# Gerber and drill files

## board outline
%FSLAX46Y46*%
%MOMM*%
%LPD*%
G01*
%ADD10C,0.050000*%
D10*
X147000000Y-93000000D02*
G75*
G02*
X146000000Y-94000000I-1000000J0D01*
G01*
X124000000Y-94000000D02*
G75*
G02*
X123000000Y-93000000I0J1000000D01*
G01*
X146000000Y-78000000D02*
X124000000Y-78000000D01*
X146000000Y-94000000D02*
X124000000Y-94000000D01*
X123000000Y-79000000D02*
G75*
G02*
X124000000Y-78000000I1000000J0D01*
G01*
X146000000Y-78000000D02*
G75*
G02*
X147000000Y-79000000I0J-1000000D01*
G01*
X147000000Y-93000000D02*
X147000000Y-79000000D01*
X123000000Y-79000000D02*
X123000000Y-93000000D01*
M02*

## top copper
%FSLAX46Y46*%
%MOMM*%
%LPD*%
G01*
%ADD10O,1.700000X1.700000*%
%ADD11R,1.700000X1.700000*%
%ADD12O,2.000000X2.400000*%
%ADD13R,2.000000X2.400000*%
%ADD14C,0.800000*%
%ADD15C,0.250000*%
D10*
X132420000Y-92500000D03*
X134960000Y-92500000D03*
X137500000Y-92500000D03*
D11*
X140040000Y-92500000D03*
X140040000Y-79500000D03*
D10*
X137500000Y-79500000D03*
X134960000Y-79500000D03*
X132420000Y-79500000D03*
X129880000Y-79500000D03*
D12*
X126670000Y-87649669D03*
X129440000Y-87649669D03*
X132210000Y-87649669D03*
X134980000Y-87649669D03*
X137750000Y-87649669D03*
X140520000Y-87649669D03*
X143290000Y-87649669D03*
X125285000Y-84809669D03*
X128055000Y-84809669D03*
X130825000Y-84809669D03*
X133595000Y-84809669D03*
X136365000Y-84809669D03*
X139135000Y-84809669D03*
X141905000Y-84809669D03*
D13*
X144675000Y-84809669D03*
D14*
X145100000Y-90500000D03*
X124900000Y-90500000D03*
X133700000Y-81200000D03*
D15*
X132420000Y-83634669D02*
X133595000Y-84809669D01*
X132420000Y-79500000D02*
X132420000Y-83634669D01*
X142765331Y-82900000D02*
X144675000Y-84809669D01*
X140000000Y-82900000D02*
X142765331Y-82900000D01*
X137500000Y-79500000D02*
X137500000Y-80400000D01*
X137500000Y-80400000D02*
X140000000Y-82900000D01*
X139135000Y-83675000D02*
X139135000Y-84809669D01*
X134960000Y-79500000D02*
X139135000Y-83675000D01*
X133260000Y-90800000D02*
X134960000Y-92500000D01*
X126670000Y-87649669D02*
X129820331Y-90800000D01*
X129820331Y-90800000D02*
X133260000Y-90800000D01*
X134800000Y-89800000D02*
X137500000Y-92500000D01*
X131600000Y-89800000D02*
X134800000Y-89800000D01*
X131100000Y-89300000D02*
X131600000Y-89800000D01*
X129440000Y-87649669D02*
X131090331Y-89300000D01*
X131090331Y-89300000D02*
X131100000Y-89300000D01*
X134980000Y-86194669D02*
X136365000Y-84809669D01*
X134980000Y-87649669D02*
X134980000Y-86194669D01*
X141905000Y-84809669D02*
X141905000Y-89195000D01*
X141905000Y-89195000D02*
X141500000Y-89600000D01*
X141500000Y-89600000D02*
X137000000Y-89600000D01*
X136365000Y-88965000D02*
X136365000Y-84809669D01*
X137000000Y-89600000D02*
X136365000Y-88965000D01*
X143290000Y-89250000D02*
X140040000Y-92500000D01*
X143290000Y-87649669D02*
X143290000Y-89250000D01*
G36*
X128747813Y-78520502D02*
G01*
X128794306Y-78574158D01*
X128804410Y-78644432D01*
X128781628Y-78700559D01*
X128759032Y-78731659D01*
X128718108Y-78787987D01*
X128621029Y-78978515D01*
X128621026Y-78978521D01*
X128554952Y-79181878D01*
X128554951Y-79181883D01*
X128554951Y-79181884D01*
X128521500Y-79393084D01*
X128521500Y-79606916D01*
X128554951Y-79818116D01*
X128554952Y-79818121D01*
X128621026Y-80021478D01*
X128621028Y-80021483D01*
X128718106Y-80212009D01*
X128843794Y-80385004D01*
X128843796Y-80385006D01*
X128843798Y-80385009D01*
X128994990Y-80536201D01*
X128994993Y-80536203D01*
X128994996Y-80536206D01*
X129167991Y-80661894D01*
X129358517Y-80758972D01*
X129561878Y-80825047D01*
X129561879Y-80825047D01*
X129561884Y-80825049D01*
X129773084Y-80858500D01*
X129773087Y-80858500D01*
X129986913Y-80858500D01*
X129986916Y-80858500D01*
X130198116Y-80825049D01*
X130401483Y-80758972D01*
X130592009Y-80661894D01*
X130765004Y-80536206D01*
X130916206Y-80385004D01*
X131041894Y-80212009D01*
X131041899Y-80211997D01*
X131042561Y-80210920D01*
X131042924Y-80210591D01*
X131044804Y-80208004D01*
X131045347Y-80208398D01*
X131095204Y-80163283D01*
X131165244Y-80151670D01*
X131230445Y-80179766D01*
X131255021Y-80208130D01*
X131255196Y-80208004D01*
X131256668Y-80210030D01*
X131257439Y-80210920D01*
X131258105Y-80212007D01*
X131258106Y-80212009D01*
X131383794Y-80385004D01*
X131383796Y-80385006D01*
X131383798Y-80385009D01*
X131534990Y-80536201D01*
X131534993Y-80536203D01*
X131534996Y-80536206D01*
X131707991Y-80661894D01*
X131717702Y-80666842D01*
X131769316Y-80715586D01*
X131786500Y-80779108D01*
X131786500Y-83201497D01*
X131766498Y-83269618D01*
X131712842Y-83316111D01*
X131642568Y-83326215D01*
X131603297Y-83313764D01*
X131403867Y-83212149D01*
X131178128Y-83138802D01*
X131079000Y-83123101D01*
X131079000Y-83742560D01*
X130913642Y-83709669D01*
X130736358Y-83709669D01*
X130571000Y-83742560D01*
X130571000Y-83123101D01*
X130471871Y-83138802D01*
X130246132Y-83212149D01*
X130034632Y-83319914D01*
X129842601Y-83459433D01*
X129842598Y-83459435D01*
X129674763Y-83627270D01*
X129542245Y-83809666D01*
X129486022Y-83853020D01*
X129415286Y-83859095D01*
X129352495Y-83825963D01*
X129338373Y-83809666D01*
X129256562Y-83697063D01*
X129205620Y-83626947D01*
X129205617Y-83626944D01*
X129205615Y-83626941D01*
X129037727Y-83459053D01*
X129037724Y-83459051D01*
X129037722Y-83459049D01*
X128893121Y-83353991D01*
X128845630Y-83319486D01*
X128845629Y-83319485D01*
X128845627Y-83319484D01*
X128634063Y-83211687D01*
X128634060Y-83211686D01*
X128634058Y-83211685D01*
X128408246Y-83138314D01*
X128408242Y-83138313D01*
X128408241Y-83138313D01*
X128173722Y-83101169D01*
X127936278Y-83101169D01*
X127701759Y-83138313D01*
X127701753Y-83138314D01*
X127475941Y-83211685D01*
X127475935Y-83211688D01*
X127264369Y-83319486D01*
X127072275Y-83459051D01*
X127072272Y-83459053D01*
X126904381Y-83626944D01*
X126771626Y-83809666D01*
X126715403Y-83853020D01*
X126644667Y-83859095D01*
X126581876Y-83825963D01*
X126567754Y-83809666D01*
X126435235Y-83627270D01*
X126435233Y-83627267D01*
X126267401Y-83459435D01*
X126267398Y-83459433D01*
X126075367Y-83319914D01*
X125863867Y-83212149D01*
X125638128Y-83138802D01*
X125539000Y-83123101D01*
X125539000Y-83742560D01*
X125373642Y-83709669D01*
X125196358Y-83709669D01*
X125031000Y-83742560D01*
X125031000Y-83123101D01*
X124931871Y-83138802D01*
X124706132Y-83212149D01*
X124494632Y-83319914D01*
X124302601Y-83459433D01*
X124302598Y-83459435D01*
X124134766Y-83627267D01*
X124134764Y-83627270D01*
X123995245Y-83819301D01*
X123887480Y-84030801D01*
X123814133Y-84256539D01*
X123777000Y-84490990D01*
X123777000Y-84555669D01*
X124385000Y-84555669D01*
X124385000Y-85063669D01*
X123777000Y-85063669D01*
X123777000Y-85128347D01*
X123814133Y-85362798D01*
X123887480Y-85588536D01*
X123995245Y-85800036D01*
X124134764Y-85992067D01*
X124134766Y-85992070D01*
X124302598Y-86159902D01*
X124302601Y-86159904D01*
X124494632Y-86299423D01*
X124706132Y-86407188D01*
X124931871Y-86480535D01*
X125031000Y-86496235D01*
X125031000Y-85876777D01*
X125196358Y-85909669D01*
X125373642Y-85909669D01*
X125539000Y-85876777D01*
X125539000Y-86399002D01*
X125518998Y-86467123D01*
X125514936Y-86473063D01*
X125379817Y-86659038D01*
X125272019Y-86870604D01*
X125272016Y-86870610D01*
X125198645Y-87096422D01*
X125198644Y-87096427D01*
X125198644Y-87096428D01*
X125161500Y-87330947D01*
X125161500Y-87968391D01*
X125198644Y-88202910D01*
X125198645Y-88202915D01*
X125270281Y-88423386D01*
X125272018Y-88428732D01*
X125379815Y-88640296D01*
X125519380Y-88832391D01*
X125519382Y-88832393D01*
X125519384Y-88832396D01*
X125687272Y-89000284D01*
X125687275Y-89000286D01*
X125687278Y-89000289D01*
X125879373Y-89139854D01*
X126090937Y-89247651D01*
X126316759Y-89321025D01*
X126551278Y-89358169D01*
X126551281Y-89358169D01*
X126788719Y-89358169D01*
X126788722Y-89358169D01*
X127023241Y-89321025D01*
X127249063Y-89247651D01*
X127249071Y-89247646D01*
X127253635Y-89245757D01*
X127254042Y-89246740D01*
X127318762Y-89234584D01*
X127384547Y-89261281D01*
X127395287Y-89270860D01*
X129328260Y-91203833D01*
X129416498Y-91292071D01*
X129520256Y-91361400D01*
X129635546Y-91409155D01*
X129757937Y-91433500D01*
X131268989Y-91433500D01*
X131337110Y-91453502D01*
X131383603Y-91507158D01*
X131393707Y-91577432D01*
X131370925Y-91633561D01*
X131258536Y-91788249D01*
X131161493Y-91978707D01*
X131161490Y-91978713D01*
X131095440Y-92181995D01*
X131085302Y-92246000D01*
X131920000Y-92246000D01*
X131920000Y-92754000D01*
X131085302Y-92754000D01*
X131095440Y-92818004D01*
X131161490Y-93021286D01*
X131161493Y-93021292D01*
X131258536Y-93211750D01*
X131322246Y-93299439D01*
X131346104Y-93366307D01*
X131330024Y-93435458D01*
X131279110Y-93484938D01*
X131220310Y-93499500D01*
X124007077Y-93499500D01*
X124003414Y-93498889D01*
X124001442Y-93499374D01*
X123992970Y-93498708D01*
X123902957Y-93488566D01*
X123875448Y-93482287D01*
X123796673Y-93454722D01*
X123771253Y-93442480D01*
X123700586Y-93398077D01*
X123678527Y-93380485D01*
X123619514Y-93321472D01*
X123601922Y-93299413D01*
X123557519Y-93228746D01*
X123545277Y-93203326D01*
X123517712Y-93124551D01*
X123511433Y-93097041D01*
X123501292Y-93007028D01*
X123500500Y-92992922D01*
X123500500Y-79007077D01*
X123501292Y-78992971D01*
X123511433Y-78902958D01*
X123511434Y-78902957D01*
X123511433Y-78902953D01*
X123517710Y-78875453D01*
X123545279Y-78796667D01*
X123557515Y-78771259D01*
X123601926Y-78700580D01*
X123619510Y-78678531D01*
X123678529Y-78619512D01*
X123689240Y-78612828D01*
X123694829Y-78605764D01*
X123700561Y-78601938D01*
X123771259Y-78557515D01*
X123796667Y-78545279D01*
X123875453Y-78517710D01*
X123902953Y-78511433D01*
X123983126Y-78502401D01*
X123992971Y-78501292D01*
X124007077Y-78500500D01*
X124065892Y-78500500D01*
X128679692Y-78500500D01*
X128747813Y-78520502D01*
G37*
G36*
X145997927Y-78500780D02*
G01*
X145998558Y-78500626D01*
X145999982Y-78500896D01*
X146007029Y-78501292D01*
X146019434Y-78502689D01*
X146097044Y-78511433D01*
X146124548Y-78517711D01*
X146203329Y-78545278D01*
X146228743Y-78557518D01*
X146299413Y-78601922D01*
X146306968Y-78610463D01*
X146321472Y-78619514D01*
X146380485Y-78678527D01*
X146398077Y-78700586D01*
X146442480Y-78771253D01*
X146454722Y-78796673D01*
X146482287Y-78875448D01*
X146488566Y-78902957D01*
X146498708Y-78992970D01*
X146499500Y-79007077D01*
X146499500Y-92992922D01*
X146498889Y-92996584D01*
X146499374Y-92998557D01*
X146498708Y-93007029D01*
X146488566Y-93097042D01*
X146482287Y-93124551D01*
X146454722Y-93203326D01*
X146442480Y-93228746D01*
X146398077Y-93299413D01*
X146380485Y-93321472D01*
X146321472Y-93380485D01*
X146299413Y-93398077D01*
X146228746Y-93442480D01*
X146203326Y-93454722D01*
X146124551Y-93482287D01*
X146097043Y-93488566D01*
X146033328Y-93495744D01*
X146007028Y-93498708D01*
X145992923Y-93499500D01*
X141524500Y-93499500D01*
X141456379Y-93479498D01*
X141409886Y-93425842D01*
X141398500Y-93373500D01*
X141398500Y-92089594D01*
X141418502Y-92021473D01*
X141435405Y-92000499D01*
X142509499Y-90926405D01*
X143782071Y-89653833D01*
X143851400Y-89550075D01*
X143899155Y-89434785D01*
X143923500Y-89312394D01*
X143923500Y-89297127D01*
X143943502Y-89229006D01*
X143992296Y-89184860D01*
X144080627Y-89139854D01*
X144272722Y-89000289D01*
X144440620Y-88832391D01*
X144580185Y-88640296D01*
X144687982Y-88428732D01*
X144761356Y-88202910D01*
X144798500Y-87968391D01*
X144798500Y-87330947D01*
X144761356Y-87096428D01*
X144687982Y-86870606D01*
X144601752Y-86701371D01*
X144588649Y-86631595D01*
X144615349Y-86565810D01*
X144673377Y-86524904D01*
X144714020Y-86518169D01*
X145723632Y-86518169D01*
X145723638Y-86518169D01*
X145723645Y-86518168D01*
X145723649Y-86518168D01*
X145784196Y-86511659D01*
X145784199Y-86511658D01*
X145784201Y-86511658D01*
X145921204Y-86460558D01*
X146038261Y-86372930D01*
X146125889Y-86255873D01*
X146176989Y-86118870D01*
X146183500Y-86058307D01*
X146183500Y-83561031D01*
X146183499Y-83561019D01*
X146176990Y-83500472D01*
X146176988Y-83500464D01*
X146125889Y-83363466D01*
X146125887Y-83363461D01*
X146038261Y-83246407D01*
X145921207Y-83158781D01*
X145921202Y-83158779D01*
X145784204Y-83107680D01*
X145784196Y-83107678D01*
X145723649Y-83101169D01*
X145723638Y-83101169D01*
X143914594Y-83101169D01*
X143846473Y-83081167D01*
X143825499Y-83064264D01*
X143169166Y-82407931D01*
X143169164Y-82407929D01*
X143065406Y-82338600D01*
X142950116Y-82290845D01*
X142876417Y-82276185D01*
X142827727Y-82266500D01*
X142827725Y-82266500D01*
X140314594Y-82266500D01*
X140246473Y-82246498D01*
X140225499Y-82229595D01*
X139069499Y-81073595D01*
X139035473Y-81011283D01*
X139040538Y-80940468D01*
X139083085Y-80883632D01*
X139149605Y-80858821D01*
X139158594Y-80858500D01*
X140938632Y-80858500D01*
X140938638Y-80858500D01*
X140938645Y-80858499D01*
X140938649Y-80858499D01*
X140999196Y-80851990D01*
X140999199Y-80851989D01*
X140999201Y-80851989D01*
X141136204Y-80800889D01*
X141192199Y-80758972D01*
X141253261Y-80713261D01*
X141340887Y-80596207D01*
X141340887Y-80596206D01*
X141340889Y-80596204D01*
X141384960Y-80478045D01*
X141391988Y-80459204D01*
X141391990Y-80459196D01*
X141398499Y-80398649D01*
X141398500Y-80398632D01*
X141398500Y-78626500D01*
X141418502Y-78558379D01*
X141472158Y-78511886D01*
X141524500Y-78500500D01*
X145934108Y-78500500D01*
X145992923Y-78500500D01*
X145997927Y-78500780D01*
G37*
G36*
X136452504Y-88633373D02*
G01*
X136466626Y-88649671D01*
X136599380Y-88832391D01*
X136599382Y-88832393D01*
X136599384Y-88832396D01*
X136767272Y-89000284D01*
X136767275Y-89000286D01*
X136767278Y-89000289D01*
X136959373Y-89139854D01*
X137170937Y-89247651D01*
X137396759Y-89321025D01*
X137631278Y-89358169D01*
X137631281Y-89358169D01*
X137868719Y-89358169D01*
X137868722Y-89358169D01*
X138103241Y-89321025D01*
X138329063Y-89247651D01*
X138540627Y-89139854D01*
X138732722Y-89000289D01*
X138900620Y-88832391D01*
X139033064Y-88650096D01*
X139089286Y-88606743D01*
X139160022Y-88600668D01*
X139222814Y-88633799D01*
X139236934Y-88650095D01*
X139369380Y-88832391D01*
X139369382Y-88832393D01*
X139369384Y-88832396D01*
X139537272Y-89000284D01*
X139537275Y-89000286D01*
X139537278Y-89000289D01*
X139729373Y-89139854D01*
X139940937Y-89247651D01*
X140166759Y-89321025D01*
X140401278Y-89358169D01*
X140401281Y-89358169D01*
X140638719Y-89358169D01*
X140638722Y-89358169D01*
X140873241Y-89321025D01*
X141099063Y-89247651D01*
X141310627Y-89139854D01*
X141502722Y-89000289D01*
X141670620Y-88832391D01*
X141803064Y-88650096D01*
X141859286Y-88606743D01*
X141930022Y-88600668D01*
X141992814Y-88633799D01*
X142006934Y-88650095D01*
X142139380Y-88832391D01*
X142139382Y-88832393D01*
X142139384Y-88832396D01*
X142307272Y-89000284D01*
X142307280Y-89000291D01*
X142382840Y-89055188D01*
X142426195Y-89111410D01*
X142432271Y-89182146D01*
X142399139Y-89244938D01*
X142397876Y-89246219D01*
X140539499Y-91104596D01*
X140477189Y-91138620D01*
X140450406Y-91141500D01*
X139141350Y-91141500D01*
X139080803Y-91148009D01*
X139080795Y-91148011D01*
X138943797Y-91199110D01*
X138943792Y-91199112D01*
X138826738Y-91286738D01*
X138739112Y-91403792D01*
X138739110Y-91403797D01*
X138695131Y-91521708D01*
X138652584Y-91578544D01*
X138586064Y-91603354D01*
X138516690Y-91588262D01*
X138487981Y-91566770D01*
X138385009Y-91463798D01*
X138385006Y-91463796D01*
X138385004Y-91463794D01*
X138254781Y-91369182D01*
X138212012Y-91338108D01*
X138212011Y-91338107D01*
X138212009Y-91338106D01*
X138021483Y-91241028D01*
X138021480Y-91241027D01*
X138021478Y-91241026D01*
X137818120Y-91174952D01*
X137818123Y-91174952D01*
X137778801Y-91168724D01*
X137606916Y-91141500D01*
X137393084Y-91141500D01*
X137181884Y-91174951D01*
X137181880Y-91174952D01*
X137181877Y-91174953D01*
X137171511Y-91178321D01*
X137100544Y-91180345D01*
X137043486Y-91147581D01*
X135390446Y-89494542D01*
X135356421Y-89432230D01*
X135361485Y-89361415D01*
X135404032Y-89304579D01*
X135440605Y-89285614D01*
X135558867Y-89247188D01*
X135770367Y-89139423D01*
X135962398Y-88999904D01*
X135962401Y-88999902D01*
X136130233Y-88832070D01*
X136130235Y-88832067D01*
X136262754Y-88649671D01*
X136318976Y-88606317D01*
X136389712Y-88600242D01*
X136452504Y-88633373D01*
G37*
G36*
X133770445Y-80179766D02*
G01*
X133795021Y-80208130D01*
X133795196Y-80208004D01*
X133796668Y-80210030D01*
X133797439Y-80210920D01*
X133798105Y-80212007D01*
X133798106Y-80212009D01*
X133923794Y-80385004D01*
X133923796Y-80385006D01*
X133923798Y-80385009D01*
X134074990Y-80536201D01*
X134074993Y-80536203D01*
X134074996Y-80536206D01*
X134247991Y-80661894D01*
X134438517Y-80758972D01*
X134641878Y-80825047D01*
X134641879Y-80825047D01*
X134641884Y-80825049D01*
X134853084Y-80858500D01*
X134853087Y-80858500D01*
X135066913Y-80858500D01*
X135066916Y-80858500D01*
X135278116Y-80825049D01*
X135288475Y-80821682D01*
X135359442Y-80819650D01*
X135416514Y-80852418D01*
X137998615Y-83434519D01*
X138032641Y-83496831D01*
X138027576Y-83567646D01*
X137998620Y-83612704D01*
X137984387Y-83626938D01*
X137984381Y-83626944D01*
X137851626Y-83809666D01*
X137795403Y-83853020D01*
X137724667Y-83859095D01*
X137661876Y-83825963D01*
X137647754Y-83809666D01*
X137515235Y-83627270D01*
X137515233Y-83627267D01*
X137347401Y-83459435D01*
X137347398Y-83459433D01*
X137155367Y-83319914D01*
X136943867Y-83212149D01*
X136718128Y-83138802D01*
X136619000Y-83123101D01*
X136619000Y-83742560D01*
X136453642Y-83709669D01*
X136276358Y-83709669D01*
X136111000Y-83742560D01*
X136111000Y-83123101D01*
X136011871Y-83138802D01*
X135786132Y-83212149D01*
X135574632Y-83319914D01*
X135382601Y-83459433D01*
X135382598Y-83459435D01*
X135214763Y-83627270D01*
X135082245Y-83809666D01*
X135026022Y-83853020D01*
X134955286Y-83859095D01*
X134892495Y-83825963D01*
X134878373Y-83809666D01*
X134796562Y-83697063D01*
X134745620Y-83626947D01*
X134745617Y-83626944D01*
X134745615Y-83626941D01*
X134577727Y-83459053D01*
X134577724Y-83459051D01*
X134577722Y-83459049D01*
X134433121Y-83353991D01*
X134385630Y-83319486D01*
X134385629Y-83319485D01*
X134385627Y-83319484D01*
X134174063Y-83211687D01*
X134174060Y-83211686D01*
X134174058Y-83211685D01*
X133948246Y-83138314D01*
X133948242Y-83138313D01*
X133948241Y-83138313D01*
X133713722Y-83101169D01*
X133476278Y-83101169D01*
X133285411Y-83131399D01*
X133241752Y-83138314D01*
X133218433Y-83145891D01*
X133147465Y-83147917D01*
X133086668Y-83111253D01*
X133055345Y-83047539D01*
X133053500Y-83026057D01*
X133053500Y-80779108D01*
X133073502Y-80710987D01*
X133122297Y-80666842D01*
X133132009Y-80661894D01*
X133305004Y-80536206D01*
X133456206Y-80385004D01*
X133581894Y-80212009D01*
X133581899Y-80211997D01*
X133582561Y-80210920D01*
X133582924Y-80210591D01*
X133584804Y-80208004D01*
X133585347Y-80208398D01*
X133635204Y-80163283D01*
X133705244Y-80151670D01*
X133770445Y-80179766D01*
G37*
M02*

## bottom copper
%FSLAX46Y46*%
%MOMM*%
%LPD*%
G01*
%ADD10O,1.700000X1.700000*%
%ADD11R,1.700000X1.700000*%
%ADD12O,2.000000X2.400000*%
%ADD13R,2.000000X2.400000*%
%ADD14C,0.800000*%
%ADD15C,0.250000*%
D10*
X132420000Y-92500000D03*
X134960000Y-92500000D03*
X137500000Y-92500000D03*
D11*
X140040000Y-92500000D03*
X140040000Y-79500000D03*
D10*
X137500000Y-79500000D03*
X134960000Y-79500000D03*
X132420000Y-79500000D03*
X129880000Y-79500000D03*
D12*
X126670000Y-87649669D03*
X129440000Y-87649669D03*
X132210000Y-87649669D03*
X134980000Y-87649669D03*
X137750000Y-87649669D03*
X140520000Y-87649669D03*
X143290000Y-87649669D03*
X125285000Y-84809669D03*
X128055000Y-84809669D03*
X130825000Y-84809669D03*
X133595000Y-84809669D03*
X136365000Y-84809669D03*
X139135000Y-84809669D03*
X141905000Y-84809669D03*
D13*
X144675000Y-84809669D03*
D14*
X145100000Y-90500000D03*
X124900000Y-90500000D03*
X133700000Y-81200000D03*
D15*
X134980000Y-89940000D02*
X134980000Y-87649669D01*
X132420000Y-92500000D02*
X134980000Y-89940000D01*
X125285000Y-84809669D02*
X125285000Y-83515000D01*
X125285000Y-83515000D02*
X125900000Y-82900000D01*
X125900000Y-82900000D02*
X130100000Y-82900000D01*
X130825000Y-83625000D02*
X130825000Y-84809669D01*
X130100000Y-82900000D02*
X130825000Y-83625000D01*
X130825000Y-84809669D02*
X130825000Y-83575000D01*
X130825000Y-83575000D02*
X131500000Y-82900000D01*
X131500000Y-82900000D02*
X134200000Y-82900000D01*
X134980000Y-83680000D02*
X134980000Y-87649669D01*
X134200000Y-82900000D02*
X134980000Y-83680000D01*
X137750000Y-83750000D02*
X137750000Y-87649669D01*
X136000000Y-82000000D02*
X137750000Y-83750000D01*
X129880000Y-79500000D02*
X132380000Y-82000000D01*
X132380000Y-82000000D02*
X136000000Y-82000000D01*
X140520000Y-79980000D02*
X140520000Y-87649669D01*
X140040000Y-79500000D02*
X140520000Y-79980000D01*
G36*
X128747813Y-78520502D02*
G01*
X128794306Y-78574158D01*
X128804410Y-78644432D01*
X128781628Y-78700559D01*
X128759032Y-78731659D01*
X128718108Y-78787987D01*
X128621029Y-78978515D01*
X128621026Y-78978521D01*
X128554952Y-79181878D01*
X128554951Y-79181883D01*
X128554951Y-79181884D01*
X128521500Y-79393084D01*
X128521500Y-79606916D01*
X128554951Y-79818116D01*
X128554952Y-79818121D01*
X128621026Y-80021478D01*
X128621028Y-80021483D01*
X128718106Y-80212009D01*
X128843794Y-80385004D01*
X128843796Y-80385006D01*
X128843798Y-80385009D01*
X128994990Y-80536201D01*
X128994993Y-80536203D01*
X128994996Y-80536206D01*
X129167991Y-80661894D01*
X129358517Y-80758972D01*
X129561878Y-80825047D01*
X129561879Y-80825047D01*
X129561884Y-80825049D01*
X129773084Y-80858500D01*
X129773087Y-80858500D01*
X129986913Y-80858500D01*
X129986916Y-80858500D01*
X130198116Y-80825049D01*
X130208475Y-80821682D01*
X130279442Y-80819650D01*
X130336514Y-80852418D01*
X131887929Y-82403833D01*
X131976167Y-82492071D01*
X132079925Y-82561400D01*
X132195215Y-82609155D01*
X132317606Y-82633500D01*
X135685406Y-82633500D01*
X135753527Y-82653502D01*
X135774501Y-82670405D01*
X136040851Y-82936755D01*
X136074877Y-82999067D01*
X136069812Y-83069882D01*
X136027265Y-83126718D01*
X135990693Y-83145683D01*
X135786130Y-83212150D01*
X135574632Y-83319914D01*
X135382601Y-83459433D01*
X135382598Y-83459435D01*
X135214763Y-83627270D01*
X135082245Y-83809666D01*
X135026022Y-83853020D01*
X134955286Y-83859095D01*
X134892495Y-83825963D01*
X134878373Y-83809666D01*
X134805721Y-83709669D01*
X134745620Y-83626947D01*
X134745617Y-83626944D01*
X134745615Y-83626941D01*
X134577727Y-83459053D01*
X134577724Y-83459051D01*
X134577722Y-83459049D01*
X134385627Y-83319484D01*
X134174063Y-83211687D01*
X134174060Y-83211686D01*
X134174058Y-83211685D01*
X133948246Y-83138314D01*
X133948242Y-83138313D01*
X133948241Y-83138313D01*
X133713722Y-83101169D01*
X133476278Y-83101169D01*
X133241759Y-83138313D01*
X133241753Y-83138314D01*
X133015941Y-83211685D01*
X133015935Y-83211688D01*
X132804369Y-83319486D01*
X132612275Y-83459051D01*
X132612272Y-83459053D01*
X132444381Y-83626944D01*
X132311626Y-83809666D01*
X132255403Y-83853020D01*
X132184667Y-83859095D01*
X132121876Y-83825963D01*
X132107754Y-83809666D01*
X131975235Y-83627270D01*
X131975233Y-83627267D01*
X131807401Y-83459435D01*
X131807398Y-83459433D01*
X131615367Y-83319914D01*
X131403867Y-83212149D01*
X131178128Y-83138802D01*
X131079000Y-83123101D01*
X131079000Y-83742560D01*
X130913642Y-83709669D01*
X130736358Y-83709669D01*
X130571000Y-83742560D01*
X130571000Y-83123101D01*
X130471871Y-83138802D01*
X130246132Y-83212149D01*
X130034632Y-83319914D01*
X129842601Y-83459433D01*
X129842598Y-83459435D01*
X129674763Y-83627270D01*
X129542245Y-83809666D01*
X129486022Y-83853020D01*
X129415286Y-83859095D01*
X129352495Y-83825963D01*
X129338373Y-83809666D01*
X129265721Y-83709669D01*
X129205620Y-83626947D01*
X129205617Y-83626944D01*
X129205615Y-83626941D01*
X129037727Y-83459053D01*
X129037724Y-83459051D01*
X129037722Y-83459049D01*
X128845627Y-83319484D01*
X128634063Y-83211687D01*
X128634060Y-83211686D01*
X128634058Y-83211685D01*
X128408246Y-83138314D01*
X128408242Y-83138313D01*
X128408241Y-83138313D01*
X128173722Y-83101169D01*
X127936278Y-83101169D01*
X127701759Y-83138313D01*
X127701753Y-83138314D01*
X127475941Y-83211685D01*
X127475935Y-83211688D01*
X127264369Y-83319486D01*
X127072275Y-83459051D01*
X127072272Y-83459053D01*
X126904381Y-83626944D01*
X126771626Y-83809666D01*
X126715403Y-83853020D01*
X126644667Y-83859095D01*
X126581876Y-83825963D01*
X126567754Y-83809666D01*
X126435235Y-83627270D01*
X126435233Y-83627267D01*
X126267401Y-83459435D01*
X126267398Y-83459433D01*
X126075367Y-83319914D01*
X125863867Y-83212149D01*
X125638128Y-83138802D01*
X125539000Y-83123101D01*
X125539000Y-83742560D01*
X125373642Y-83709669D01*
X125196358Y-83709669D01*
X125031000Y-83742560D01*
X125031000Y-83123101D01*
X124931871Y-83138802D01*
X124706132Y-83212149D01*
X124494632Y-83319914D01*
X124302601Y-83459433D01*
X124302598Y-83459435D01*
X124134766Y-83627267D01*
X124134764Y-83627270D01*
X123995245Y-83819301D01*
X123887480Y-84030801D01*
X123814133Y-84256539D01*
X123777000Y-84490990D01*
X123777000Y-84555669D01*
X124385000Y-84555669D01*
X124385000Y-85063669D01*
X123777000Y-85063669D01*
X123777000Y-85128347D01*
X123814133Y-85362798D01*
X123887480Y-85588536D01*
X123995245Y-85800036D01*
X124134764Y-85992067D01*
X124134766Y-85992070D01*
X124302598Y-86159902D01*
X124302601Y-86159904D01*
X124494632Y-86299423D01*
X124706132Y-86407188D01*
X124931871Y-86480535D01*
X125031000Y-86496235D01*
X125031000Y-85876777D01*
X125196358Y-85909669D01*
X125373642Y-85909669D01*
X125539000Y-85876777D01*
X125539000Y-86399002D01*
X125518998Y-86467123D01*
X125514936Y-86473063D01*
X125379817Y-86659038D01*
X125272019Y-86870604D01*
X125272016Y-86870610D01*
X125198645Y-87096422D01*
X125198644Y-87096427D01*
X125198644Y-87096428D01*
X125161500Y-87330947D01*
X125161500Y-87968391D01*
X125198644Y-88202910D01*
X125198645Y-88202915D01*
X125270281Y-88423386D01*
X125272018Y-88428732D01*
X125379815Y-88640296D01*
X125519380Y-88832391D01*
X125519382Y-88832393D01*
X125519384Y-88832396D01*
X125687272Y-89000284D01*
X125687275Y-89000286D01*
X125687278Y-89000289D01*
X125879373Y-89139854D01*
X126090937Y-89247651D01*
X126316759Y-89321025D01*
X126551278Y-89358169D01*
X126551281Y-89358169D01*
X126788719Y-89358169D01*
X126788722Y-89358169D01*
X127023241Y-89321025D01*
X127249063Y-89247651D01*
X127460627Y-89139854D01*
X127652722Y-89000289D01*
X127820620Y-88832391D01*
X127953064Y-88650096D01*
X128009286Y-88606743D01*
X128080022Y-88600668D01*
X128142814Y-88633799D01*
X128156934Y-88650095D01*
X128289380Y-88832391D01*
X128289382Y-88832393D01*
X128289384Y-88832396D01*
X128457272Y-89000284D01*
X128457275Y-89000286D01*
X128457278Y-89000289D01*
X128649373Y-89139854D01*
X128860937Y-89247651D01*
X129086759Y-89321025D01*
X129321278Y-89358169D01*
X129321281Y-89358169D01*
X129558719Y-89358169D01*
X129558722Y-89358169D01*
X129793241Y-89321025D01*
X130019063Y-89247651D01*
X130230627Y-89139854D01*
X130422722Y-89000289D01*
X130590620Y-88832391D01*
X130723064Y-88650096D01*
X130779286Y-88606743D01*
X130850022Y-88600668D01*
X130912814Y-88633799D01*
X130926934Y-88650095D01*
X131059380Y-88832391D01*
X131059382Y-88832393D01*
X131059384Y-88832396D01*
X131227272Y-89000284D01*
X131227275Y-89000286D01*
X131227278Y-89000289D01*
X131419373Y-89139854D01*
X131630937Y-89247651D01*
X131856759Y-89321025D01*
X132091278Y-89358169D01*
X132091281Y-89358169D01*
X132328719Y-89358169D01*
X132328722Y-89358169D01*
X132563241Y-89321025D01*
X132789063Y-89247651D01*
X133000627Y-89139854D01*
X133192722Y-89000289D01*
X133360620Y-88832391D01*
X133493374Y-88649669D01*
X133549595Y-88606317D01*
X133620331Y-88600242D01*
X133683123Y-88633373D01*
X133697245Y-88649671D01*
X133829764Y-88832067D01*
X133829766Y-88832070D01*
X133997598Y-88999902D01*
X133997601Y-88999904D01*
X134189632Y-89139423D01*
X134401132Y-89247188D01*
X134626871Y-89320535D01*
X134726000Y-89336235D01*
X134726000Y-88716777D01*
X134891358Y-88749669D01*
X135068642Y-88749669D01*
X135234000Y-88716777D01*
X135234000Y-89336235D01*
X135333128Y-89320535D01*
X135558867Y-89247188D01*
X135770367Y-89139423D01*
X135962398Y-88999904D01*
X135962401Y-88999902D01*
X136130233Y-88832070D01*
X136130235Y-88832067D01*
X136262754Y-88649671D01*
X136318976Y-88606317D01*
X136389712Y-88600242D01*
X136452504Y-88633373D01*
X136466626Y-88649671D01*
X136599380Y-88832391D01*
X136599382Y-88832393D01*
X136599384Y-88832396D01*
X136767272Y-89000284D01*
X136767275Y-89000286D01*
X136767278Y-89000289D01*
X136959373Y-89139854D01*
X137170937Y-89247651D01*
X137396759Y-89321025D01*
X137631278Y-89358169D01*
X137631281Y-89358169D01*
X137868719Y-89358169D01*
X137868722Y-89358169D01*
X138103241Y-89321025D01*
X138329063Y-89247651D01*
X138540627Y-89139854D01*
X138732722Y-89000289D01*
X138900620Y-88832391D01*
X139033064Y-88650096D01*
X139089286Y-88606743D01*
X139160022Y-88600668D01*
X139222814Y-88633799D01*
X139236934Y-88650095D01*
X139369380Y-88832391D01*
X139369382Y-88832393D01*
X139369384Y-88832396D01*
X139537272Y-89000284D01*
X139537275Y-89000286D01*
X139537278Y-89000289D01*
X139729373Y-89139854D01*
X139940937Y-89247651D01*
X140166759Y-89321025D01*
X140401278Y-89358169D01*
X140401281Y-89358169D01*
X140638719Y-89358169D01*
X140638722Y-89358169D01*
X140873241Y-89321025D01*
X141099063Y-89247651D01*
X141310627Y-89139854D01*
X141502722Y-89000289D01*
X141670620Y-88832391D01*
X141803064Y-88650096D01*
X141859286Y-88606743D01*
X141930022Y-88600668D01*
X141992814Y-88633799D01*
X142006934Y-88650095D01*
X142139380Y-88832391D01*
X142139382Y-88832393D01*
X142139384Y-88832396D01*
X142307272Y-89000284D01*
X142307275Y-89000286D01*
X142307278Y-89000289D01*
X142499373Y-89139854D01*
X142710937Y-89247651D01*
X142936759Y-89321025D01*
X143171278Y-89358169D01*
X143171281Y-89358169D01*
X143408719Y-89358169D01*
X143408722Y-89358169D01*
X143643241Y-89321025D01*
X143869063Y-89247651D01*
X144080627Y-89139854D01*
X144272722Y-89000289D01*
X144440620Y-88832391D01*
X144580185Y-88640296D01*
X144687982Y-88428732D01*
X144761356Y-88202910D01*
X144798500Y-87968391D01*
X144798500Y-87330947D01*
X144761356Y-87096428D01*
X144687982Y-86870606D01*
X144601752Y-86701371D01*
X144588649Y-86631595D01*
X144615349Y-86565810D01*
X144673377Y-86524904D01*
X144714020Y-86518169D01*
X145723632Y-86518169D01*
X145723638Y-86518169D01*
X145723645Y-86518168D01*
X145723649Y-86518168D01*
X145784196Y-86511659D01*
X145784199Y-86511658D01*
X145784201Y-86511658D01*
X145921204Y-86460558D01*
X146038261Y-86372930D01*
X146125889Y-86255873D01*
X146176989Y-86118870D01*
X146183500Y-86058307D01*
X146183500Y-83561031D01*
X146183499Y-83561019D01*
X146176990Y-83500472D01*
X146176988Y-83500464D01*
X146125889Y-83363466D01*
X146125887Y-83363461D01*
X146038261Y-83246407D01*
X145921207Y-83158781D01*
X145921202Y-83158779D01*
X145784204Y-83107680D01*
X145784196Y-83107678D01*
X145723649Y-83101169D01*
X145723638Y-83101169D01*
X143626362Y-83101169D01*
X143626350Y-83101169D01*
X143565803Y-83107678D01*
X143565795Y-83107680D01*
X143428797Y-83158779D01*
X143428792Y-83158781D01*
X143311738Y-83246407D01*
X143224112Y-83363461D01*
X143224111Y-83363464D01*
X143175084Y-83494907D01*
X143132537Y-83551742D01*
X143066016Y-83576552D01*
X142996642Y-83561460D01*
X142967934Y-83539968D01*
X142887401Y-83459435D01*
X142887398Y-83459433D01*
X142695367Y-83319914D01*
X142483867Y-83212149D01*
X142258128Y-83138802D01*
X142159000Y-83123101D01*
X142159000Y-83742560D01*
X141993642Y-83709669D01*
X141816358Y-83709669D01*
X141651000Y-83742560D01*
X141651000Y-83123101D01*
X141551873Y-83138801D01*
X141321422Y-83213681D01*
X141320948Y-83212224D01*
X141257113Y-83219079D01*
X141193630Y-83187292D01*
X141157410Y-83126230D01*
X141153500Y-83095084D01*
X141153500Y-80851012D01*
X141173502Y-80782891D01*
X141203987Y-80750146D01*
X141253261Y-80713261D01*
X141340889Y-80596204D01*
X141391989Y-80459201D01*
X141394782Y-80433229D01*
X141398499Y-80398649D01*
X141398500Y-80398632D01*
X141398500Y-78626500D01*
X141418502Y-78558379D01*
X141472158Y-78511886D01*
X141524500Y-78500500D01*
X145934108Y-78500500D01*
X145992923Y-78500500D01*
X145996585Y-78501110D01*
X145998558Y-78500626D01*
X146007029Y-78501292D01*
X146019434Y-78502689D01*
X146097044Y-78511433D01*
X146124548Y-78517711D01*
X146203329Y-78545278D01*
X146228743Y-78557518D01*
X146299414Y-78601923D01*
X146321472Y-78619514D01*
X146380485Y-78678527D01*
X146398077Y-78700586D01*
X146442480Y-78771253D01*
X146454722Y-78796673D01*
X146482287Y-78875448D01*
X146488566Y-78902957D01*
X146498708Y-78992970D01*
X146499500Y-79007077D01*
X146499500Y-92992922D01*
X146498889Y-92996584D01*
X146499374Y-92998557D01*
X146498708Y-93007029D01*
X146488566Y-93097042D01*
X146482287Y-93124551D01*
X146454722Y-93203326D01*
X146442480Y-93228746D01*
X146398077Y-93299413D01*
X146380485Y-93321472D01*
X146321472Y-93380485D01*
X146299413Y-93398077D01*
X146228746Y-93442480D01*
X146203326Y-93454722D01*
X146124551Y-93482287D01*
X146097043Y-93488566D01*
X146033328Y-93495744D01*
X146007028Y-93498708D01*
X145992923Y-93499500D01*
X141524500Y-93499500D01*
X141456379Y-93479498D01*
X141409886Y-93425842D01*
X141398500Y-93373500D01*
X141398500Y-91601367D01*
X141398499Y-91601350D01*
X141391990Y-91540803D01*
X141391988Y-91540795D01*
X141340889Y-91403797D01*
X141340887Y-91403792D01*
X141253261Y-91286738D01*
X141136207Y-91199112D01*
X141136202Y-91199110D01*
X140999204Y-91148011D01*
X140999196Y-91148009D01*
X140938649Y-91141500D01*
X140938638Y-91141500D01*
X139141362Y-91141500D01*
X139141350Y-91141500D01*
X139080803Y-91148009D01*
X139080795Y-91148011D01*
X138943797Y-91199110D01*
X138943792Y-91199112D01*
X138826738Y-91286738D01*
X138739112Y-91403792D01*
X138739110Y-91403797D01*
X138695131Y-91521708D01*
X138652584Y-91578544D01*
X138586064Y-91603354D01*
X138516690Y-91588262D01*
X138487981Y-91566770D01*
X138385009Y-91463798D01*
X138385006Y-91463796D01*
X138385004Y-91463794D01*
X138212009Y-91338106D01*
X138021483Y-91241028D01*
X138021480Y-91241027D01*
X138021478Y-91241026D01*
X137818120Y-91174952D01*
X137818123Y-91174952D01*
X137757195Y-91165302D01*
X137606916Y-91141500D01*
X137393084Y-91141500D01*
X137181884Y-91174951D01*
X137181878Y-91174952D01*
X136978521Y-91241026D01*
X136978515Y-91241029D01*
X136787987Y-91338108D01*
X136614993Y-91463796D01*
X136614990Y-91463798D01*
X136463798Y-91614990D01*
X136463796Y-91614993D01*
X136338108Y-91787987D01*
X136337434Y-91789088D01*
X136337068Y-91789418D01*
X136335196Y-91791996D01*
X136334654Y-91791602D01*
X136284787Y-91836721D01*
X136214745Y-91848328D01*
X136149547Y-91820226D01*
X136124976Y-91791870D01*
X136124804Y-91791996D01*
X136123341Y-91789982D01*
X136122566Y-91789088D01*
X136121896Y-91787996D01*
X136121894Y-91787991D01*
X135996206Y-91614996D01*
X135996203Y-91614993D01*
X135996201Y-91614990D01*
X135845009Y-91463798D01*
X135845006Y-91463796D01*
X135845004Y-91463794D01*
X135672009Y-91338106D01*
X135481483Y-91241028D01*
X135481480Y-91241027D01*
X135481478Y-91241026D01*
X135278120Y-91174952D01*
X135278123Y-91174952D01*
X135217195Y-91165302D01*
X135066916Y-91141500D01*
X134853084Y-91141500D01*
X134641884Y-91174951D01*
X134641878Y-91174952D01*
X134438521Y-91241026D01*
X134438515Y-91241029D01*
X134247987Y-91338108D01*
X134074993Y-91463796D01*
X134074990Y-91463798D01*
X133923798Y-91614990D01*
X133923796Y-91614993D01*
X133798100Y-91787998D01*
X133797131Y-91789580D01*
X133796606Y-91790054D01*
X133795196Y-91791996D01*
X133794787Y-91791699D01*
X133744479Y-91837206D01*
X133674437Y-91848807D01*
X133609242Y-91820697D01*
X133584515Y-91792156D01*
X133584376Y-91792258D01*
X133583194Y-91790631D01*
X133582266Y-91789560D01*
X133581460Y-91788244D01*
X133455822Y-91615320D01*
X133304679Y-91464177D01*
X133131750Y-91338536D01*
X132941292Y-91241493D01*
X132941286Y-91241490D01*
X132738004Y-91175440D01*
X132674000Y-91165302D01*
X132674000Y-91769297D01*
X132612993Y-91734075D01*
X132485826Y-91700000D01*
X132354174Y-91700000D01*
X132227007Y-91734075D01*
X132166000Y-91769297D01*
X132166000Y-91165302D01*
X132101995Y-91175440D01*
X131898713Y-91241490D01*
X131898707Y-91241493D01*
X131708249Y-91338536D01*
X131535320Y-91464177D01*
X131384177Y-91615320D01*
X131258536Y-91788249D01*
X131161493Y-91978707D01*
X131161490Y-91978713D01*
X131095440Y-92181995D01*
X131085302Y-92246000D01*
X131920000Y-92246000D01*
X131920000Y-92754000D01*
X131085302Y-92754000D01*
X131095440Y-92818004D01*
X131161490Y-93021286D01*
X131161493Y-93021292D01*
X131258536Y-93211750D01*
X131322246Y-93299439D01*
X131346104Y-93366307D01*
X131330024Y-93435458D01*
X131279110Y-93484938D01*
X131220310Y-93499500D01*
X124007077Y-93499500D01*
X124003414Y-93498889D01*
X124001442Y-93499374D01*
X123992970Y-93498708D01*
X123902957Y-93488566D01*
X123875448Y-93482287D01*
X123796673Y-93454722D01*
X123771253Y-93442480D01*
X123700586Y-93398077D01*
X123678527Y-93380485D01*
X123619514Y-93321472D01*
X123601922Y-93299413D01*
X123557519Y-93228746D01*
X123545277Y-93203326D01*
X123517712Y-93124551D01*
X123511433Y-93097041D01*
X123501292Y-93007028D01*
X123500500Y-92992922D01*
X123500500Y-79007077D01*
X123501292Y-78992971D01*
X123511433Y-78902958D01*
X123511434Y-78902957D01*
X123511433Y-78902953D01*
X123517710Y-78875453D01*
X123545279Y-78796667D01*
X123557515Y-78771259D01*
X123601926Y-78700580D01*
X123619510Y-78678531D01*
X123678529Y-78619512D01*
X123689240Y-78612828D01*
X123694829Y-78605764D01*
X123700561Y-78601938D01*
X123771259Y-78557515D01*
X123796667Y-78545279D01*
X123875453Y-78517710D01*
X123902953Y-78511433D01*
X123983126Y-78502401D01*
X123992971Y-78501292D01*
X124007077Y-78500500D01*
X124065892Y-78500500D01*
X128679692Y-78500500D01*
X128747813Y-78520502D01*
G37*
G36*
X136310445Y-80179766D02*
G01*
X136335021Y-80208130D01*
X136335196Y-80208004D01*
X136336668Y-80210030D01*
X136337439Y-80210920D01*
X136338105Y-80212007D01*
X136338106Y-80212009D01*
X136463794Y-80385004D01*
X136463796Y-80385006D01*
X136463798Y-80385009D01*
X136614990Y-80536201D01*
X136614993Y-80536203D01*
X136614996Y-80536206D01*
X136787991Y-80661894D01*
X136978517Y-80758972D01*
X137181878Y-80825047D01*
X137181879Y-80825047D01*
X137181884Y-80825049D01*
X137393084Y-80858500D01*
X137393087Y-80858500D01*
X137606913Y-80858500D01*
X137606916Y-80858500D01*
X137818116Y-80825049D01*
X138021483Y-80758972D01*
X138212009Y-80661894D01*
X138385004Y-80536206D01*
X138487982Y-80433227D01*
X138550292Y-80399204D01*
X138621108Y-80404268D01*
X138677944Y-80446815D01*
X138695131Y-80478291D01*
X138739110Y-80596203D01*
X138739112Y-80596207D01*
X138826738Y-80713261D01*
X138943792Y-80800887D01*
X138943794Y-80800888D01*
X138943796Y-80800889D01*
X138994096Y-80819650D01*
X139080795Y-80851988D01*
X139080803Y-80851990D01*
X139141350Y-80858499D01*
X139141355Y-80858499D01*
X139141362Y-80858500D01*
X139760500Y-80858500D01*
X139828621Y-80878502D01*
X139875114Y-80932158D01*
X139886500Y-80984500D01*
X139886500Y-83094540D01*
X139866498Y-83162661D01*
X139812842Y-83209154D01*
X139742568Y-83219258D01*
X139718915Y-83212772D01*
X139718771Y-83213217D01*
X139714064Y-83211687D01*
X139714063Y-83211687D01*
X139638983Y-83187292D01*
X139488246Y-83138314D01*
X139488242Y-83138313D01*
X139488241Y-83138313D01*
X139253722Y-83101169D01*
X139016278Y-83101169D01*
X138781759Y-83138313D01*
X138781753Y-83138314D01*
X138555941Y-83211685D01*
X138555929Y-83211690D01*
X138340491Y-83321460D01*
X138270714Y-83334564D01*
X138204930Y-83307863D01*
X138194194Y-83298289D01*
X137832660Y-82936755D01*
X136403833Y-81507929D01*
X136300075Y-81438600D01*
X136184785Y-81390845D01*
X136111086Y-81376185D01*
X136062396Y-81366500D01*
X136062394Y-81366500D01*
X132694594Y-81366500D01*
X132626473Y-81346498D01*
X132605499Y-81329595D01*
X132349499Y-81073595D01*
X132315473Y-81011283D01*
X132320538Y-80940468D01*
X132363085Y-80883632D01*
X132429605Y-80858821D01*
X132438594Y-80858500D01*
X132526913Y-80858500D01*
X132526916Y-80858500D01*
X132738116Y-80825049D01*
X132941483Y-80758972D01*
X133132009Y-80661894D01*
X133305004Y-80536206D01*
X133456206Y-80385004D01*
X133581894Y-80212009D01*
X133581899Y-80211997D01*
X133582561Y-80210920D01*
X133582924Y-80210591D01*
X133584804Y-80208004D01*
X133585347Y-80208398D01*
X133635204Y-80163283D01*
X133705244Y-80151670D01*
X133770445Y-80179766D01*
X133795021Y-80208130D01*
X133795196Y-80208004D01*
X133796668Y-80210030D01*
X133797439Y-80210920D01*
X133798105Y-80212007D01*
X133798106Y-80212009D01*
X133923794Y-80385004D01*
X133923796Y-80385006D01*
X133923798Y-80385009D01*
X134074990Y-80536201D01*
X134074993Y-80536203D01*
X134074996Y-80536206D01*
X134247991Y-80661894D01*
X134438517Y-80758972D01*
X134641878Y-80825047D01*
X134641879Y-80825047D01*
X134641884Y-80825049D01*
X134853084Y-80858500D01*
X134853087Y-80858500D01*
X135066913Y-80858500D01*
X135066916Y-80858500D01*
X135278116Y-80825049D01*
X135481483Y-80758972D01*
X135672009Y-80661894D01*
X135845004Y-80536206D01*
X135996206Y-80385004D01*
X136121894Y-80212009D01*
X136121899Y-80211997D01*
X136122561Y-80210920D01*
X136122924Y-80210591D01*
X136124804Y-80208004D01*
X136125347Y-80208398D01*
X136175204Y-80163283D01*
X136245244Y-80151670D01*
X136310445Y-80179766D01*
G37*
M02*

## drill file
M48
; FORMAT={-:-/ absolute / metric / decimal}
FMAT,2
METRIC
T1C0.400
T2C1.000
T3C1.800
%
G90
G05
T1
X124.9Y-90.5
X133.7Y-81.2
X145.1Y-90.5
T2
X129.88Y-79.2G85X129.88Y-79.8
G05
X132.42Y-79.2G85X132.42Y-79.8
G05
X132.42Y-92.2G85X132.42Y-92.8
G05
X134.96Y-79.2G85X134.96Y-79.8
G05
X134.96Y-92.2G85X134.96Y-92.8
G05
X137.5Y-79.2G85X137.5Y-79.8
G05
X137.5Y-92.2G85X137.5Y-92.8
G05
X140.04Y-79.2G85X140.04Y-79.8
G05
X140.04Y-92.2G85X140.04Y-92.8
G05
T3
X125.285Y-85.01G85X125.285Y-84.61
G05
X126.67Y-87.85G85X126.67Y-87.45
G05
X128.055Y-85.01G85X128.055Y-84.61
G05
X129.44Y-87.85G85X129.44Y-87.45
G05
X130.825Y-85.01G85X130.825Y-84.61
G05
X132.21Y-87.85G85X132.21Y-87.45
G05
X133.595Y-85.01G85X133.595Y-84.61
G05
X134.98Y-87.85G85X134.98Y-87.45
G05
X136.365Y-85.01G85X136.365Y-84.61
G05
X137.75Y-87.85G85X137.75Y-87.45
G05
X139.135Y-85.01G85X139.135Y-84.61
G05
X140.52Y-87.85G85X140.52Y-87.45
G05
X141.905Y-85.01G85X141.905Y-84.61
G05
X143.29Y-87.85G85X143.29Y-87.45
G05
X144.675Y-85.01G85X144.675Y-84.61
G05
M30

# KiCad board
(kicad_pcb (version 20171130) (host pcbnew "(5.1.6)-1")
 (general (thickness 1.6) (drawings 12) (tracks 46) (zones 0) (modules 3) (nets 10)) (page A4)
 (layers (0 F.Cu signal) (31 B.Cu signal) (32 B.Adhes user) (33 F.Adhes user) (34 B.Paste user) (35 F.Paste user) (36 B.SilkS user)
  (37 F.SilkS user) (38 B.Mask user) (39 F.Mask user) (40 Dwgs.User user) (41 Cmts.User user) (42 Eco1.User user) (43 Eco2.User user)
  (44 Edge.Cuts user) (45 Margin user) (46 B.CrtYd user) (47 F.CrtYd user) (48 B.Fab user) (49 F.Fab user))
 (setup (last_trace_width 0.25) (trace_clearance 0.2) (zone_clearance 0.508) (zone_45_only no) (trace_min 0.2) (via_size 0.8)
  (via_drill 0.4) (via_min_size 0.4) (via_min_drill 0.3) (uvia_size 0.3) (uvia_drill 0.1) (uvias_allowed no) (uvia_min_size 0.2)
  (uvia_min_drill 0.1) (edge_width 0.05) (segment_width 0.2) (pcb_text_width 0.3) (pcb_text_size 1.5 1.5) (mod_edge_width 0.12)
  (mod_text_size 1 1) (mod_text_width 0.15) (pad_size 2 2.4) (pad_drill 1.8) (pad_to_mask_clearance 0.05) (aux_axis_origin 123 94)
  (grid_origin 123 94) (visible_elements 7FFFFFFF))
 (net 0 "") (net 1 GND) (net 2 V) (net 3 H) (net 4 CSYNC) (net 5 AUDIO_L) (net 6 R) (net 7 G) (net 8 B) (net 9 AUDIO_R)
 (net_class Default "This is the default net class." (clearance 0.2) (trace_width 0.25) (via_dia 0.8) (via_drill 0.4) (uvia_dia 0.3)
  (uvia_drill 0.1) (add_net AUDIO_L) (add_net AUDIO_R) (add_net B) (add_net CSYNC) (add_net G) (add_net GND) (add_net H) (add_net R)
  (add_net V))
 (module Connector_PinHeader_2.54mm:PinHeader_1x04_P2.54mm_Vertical (layer F.Cu) (at 140.04 92.5 270)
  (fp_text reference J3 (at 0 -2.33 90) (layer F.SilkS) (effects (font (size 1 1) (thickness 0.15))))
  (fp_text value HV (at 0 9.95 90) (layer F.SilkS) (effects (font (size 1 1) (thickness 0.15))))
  (pad 4 thru_hole oval (at 0 7.62 270) (size 1.7 1.7) (drill oval 1.6 1) (layers *.Cu *.Mask) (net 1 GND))
  (pad 3 thru_hole oval (at 0 5.08 270) (size 1.7 1.7) (drill oval 1.6 1) (layers *.Cu *.Mask) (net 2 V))
  (pad 2 thru_hole oval (at 0 2.54 270) (size 1.7 1.7) (drill oval 1.6 1) (layers *.Cu *.Mask) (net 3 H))
  (pad 1 thru_hole rect (at 0 0 270) (size 1.7 1.7) (drill oval 1.6 1) (layers *.Cu *.Mask) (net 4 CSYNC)))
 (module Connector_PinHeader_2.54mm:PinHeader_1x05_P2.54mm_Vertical (layer F.Cu) (at 140.04 79.5 270)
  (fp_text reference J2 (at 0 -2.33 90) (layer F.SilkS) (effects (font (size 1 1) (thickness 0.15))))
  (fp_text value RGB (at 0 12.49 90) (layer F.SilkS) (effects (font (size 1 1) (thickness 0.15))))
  (pad 1 thru_hole rect (at 0 0 270) (size 1.7 1.7) (drill oval 1.6 1) (layers *.Cu *.Mask) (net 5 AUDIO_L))
  (pad 2 thru_hole oval (at 0 2.54 270) (size 1.7 1.7) (drill oval 1.6 1) (layers *.Cu *.Mask) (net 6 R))
  (pad 3 thru_hole oval (at 0 5.08 270) (size 1.7 1.7) (drill oval 1.6 1) (layers *.Cu *.Mask) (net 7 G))
  (pad 4 thru_hole oval (at 0 7.62 270) (size 1.7 1.7) (drill oval 1.6 1) (layers *.Cu *.Mask) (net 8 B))
  (pad 5 thru_hole oval (at 0 10.16 270) (size 1.7 1.7) (drill oval 1.6 1) (layers *.Cu *.Mask) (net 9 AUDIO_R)))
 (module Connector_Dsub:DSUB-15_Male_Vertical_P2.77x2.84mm (layer B.Cu) (at 144.675 84.809669 180)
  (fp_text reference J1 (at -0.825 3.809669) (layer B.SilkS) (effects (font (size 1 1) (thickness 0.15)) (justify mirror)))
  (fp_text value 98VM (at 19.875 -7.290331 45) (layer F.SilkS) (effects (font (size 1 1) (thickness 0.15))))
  (pad 15 thru_hole oval (at 18.005 -2.84 180) (size 2 2.4) (drill oval 1.8 2.2) (layers *.Cu *.Mask) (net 2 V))
  (pad 14 thru_hole oval (at 15.235 -2.84 180) (size 2 2.4) (drill oval 1.8 2.2) (layers *.Cu *.Mask) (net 3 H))
  (pad 13 thru_hole oval (at 12.465 -2.84 180) (size 2 2.4) (drill oval 1.8 2.2) (layers *.Cu *.Mask))
  (pad 12 thru_hole oval (at 9.695 -2.84 180) (size 2 2.4) (drill oval 1.8 2.2) (layers *.Cu *.Mask) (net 1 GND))
  (pad 11 thru_hole oval (at 6.925 -2.84 180) (size 2 2.4) (drill oval 1.8 2.2) (layers *.Cu *.Mask) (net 9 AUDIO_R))
  (pad 10 thru_hole oval (at 4.155 -2.84 180) (size 2 2.4) (drill oval 1.8 2.2) (layers *.Cu *.Mask) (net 5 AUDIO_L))
  (pad 9 thru_hole oval (at 1.385 -2.84 180) (size 2 2.4) (drill oval 1.8 2.2) (layers *.Cu *.Mask) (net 4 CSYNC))
  (pad 8 thru_hole oval (at 19.39 0 180) (size 2 2.4) (drill oval 1.8 2.2) (layers *.Cu *.Mask) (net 1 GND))
  (pad 7 thru_hole oval (at 16.62 0 180) (size 2 2.4) (drill oval 1.8 2.2) (layers *.Cu *.Mask))
  (pad 6 thru_hole oval (at 13.85 0 180) (size 2 2.4) (drill oval 1.8 2.2) (layers *.Cu *.Mask) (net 1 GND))
  (pad 5 thru_hole oval (at 11.08 0 180) (size 2 2.4) (drill oval 1.8 2.2) (layers *.Cu *.Mask) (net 8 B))
  (pad 4 thru_hole oval (at 8.31 0 180) (size 2 2.4) (drill oval 1.8 2.2) (layers *.Cu *.Mask) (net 1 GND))
  (pad 3 thru_hole oval (at 5.54 0 180) (size 2 2.4) (drill oval 1.8 2.2) (layers *.Cu *.Mask) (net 7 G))
  (pad 2 thru_hole oval (at 2.77 0 180) (size 2 2.4) (drill oval 1.8 2.2) (layers *.Cu *.Mask) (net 1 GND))
  (pad 1 thru_hole rect (at 0 0 180) (size 2 2.4) (drill oval 1.8 2.2) (layers *.Cu *.Mask) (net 6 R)))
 (gr_arc (start 146 93) (end 146 94) (angle -90) (layer Edge.Cuts) (width 0.05))
 (gr_arc (start 124 93) (end 123 93) (angle -90) (layer Edge.Cuts) (width 0.05))
 (gr_line (start 146 78) (end 124 78) (layer Edge.Cuts) (width 0.05))
 (gr_line (start 146 94) (end 124 94) (layer Edge.Cuts) (width 0.05))
 (gr_arc (start 124 79) (end 124 78) (angle -90) (layer Edge.Cuts) (width 0.05))
 (gr_arc (start 146 79) (end 147 79) (angle -90) (layer Edge.Cuts) (width 0.05))
 (gr_line (start 147 93) (end 147 79) (layer Edge.Cuts) (width 0.05))
 (gr_line (start 123 79) (end 123 93) (layer Edge.Cuts) (width 0.05))
 (segment (start 132.42 83.634669) (end 133.595 84.809669) (width 0.25) (layer F.Cu) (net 8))
 (segment (start 132.42 79.5) (end 132.42 83.634669) (width 0.25) (layer F.Cu) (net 8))
 (segment (start 142.765331 82.9) (end 144.675 84.809669) (width 0.25) (layer F.Cu) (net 6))
 (segment (start 140 82.9) (end 142.765331 82.9) (width 0.25) (layer F.Cu) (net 6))
 (segment (start 137.5 79.5) (end 137.5 80.4) (width 0.25) (layer F.Cu) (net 6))
 (segment (start 137.5 80.4) (end 140 82.9) (width 0.25) (layer F.Cu) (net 6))
 (segment (start 139.135 83.675) (end 139.135 84.809669) (width 0.25) (layer F.Cu) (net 7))
 (segment (start 134.96 79.5) (end 139.135 83.675) (width 0.25) (layer F.Cu) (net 7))
 (segment (start 133.26 90.8) (end 134.96 92.5) (width 0.25) (layer F.Cu) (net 2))
 (segment (start 126.67 87.649669) (end 129.820331 90.8) (width 0.25) (layer F.Cu) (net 2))
 (segment (start 129.820331 90.8) (end 133.26 90.8) (width 0.25) (layer F.Cu) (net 2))
 (segment (start 134.8 89.8) (end 137.5 92.5) (width 0.25) (layer F.Cu) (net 3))
 (segment (start 131.6 89.8) (end 134.8 89.8) (width 0.25) (layer F.Cu) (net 3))
 (segment (start 131.1 89.3) (end 131.6 89.8) (width 0.25) (layer F.Cu) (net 3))
 (segment (start 129.44 87.649669) (end 131.090331 89.3) (width 0.25) (layer F.Cu) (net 3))
 (segment (start 131.090331 89.3) (end 131.1 89.3) (width 0.25) (layer F.Cu) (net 3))
 (segment (start 134.98 86.194669) (end 136.365 84.809669) (width 0.25) (layer F.Cu) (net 1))
 (segment (start 134.98 87.649669) (end 134.98 86.194669) (width 0.25) (layer F.Cu) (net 1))
 (segment (start 134.98 89.94) (end 134.98 87.649669) (width 0.25) (layer B.Cu) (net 1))
 (segment (start 132.42 92.5) (end 134.98 89.94) (width 0.25) (layer B.Cu) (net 1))
 (segment (start 125.285 84.809669) (end 125.285 83.515) (width 0.25) (layer B.Cu) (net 1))
 (segment (start 125.285 83.515) (end 125.9 82.9) (width 0.25) (layer B.Cu) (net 1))
 (segment (start 125.9 82.9) (end 130.1 82.9) (width 0.25) (layer B.Cu) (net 1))
 (segment (start 130.825 83.625) (end 130.825 84.809669) (width 0.25) (layer B.Cu) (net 1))
 (segment (start 130.1 82.9) (end 130.825 83.625) (width 0.25) (layer B.Cu) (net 1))
 (segment (start 130.825 84.809669) (end 130.825 83.575) (width 0.25) (layer B.Cu) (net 1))
 (segment (start 130.825 83.575) (end 131.5 82.9) (width 0.25) (layer B.Cu) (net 1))
 (segment (start 131.5 82.9) (end 134.2 82.9) (width 0.25) (layer B.Cu) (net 1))
 (segment (start 134.98 83.68) (end 134.98 87.649669) (width 0.25) (layer B.Cu) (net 1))
 (segment (start 134.2 82.9) (end 134.98 83.68) (width 0.25) (layer B.Cu) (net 1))
 (segment (start 141.905 84.809669) (end 141.905 89.195) (width 0.25) (layer F.Cu) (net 1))
 (segment (start 141.905 89.195) (end 141.5 89.6) (width 0.25) (layer F.Cu) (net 1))
 (segment (start 141.5 89.6) (end 137 89.6) (width 0.25) (layer F.Cu) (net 1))
 (segment (start 136.365 88.965) (end 136.365 84.809669) (width 0.25) (layer F.Cu) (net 1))
 (segment (start 137 89.6) (end 136.365 88.965) (width 0.25) (layer F.Cu) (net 1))
 (via (at 145.1 90.5) (size 0.8) (drill 0.4) (layers F.Cu B.Cu) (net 1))
 (via (at 124.9 90.5) (size 0.8) (drill 0.4) (layers F.Cu B.Cu) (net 1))
 (via (at 133.7 81.2) (size 0.8) (drill 0.4) (layers F.Cu B.Cu) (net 1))
 (segment (start 137.75 83.75) (end 137.75 87.649669) (width 0.25) (layer B.Cu) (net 9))
 (segment (start 136 82) (end 137.75 83.75) (width 0.25) (layer B.Cu) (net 9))
 (segment (start 129.88 79.5) (end 132.38 82) (width 0.25) (layer B.Cu) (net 9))
 (segment (start 132.38 82) (end 136 82) (width 0.25) (layer B.Cu) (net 9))
 (segment (start 140.52 79.98) (end 140.52 87.649669) (width 0.25) (layer B.Cu) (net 5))
 (segment (start 140.04 79.5) (end 140.52 79.98) (width 0.25) (layer B.Cu) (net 5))
 (segment (start 143.29 89.25) (end 140.04 92.5) (width 0.25) (layer F.Cu) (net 4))
 (segment (start 143.29 87.649669) (end 143.29 89.25) (width 0.25) (layer F.Cu) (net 4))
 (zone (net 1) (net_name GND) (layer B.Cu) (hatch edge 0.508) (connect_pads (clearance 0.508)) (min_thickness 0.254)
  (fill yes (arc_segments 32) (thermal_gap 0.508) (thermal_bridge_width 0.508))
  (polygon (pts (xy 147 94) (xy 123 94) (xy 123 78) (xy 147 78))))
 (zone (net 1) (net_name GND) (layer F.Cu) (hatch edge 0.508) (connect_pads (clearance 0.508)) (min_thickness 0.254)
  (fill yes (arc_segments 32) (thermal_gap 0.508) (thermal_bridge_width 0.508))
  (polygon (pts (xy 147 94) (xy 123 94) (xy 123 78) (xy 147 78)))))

